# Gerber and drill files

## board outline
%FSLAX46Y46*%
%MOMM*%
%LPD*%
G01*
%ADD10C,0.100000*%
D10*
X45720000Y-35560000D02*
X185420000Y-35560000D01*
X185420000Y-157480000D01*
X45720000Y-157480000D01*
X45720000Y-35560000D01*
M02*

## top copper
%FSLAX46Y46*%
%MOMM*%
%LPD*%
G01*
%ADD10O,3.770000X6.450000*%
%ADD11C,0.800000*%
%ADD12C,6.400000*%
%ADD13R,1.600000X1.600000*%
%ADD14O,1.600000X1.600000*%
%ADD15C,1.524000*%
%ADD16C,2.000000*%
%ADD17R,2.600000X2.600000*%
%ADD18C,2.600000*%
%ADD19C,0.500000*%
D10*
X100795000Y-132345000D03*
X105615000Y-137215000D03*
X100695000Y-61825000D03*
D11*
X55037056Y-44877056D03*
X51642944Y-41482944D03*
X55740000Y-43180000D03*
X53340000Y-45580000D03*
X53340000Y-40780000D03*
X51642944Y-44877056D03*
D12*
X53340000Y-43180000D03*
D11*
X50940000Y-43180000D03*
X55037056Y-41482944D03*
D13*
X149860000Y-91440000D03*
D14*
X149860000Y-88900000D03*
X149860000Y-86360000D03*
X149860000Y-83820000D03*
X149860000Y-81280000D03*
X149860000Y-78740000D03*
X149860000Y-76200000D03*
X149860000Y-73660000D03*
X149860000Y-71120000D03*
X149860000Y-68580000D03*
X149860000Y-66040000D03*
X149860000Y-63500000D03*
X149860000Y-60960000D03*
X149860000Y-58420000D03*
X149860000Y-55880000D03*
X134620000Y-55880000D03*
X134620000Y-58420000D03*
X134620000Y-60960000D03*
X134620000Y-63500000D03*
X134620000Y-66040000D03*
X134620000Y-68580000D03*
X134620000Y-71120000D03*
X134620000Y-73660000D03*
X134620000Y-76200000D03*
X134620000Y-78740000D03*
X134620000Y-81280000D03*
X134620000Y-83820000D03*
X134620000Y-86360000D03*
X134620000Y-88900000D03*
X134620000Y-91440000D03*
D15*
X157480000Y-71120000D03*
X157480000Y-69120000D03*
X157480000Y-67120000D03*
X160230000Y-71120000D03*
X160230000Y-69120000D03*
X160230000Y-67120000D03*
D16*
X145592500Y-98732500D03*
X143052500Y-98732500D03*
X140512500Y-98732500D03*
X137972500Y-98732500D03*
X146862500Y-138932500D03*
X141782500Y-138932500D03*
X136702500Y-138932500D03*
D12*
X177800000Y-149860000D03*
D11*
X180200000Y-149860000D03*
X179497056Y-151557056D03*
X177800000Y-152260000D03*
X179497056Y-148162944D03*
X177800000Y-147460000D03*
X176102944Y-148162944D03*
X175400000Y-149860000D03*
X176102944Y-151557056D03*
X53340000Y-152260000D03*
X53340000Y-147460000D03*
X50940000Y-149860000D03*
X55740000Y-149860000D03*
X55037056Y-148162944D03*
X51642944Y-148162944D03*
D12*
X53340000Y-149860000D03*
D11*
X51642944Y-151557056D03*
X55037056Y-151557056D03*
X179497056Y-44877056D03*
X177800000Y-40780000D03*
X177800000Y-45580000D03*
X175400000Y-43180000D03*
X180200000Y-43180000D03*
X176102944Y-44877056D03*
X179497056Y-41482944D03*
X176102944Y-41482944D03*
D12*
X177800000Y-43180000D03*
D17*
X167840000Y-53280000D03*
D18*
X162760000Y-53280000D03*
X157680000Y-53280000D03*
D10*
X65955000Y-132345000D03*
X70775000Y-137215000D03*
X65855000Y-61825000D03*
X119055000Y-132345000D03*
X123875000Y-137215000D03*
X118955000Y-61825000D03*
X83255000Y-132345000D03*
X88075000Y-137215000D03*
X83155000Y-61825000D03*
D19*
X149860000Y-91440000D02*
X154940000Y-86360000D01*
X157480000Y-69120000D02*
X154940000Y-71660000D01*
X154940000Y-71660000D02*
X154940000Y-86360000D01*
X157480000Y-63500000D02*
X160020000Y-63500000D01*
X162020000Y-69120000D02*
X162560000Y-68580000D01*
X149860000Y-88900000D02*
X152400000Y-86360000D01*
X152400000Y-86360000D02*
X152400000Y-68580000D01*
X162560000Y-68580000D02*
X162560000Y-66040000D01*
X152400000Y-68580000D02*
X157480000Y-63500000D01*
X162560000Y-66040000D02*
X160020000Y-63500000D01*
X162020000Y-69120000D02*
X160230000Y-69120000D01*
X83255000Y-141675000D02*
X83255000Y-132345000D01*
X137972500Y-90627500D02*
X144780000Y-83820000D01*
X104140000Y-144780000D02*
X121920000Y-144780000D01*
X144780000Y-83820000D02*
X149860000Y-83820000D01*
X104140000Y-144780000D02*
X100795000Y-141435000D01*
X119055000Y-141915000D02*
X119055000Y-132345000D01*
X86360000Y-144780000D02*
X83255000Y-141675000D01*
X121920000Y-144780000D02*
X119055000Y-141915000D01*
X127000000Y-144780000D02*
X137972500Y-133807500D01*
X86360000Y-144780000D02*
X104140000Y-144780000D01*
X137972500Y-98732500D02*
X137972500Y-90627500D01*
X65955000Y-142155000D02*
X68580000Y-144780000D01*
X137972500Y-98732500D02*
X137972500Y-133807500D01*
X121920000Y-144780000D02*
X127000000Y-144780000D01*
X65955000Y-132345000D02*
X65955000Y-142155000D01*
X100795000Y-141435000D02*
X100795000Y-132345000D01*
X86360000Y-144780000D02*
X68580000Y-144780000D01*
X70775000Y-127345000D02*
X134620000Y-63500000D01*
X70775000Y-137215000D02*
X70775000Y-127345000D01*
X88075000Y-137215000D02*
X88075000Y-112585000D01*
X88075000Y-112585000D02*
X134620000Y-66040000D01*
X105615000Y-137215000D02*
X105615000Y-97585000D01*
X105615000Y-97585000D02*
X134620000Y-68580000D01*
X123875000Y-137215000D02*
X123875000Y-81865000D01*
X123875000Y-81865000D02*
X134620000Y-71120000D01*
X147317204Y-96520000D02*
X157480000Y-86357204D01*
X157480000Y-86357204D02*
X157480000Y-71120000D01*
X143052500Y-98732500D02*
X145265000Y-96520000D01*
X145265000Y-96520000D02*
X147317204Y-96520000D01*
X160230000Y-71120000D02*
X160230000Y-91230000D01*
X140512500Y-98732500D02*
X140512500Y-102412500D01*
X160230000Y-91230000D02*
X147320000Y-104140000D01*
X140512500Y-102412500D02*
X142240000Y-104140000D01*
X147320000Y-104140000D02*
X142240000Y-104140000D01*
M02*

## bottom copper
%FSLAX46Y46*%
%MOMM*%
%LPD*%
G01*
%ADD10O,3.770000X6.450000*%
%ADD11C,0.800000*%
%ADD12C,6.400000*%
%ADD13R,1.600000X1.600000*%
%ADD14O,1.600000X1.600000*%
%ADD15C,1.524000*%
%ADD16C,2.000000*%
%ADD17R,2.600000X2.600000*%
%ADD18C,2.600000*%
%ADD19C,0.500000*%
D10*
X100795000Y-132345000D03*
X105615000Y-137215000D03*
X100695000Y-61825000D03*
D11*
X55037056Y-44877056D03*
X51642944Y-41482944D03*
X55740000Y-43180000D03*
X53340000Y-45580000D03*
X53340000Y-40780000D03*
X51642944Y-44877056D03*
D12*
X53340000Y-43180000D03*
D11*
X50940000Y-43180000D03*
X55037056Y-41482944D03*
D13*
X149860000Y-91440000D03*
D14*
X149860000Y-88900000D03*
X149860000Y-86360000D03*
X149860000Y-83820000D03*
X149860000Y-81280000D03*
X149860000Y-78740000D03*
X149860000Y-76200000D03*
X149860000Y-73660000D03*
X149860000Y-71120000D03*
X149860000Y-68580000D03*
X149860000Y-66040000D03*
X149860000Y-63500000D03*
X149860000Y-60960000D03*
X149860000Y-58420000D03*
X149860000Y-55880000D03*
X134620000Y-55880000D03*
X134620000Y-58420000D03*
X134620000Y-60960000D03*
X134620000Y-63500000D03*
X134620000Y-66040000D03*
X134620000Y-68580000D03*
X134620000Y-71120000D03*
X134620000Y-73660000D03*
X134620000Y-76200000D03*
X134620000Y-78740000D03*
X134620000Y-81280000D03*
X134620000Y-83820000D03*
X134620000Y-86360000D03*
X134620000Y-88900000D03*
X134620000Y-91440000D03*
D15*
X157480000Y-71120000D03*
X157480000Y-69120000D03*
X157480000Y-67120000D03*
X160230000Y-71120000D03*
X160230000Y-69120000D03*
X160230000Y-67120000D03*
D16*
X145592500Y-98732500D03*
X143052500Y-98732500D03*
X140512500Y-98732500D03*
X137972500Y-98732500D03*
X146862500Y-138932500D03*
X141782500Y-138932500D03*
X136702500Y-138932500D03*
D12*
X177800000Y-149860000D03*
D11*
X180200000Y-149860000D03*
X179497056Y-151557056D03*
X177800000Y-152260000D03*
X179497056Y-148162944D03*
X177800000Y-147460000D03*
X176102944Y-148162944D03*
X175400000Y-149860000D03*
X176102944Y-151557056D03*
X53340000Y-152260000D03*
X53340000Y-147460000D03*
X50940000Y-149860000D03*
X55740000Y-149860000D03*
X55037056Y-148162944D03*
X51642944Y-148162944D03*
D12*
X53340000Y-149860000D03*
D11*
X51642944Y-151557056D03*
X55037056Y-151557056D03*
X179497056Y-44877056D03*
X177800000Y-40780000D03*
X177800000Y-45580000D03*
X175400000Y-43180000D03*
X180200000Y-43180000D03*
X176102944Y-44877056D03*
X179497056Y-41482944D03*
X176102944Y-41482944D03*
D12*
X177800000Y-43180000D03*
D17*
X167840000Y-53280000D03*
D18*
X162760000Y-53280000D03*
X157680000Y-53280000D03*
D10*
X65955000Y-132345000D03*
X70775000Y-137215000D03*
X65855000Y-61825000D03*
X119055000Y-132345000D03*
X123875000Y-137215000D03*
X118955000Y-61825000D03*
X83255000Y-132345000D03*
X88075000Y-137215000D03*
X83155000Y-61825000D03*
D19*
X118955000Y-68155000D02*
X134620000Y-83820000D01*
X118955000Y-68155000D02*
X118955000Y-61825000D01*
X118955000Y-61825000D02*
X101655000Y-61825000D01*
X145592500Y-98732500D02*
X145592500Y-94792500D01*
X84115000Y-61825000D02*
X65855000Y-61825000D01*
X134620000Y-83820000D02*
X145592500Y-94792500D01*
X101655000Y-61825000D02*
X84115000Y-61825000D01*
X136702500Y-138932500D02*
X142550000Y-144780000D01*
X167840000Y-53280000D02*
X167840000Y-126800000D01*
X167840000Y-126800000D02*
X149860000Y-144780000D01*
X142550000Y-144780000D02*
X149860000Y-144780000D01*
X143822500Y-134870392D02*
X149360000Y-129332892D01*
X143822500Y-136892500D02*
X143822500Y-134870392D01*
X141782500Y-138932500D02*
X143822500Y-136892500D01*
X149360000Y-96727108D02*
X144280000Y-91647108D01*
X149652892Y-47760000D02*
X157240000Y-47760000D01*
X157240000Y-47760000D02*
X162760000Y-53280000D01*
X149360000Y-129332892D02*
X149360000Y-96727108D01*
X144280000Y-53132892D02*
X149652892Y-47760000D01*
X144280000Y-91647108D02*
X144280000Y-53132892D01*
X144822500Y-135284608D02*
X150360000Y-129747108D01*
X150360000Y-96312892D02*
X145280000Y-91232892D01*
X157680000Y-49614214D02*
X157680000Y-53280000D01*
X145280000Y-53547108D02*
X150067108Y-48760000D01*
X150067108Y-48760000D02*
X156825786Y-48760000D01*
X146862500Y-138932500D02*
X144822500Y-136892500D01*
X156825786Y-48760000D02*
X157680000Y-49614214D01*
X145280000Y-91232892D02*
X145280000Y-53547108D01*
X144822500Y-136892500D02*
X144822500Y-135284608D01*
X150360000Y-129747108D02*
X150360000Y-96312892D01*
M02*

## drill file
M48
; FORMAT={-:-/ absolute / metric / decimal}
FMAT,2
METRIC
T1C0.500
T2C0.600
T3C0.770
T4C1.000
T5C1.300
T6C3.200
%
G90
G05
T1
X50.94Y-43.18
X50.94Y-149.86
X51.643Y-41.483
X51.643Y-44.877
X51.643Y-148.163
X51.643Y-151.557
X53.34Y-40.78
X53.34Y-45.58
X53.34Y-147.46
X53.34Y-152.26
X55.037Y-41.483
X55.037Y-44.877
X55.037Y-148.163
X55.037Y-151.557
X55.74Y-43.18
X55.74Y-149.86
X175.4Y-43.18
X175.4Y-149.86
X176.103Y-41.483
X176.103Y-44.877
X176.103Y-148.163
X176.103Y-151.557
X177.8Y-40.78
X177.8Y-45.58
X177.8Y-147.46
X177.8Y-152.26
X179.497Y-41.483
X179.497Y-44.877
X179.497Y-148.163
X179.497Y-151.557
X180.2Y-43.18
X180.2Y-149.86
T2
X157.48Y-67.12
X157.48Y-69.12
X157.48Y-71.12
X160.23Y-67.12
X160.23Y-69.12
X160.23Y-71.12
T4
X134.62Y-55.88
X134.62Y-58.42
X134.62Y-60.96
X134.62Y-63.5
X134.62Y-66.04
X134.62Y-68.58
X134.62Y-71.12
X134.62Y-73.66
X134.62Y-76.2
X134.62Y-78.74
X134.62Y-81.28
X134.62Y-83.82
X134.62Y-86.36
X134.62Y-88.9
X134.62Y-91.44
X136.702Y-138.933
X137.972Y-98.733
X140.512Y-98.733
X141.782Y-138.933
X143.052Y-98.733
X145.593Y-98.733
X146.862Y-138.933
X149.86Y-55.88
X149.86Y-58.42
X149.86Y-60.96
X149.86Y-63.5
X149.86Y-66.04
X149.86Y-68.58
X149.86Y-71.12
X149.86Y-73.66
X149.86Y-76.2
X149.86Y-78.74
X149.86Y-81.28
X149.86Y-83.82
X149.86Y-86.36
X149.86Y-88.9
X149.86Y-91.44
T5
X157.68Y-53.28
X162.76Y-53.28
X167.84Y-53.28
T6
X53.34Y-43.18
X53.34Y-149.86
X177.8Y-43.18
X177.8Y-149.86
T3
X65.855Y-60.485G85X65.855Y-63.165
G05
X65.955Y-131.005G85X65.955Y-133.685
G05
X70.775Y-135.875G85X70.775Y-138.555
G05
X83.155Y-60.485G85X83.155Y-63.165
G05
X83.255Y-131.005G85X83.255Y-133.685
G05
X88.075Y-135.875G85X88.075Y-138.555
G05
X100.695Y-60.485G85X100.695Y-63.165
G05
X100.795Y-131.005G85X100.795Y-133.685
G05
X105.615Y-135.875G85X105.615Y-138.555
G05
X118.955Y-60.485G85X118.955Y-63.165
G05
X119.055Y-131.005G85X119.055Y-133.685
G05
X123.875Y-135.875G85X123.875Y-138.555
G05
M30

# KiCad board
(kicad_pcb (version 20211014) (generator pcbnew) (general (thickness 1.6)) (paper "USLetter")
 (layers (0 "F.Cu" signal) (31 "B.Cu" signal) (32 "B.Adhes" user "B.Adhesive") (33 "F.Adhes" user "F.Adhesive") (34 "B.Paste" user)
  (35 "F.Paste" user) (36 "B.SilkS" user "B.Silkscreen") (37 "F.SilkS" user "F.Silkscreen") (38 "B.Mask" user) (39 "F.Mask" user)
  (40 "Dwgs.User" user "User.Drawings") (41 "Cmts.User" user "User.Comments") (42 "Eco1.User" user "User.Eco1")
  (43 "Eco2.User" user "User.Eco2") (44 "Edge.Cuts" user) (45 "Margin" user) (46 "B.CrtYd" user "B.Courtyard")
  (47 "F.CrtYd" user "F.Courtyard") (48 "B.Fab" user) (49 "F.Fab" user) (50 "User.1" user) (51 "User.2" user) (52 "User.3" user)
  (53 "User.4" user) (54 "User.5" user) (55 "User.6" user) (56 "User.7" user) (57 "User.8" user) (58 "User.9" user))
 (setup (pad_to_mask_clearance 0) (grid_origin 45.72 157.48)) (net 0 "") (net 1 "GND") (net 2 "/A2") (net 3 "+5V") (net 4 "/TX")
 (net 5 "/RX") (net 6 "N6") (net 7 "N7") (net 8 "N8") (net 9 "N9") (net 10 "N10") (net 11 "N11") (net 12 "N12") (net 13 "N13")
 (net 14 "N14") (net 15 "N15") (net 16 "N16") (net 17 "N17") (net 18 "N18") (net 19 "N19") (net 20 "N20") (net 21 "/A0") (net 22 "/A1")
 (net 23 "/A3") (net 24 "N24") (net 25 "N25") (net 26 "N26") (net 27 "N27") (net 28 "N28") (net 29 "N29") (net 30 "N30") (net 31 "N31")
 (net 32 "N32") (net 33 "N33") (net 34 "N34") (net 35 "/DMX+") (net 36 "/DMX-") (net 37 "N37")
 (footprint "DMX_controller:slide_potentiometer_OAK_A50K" (layer "F.Cu") (at 96.225 52.345)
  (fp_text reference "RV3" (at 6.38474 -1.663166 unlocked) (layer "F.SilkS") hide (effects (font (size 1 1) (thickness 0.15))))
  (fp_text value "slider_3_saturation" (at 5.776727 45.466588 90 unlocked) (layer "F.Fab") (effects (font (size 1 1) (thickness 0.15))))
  (pad "1" thru_hole oval (at 4.57 80) (size 3.77 6.45) (drill oval 0.77 3.45) (layers *.Cu *.Mask) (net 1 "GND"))
  (pad "2" thru_hole oval (at 9.39 84.87) (size 3.77 6.45) (drill oval 0.77 3.45) (layers *.Cu *.Mask) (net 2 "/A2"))
  (pad "3" thru_hole oval (at 4.47 9.48) (size 3.77 6.45) (drill oval 0.77 3.45) (layers *.Cu *.Mask) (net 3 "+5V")))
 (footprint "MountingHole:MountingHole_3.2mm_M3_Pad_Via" (layer "F.Cu") (at 53.34 43.18)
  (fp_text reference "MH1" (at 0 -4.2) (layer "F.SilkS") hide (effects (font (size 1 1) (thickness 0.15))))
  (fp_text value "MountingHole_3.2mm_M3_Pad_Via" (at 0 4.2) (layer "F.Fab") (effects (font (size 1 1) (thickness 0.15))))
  (pad "1" thru_hole circle (at 1.697056 1.697056) (size 0.8 0.8) (drill 0.5) (layers *.Cu *.Mask))
  (pad "1" thru_hole circle (at -1.697056 -1.697056) (size 0.8 0.8) (drill 0.5) (layers *.Cu *.Mask))
  (pad "1" thru_hole circle (at 2.4 0) (size 0.8 0.8) (drill 0.5) (layers *.Cu *.Mask))
  (pad "1" thru_hole circle (at 0 2.4) (size 0.8 0.8) (drill 0.5) (layers *.Cu *.Mask))
  (pad "1" thru_hole circle (at 0 -2.4) (size 0.8 0.8) (drill 0.5) (layers *.Cu *.Mask))
  (pad "1" thru_hole circle (at -1.697056 1.697056) (size 0.8 0.8) (drill 0.5) (layers *.Cu *.Mask))
  (pad "1" thru_hole circle (at 0 0) (size 6.4 6.4) (drill 3.2) (layers *.Cu *.Mask))
  (pad "1" thru_hole circle (at -2.4 0) (size 0.8 0.8) (drill 0.5) (layers *.Cu *.Mask))
  (pad "1" thru_hole circle (at 1.697056 -1.697056) (size 0.8 0.8) (drill 0.5) (layers *.Cu *.Mask)))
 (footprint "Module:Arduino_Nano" (layer "F.Cu") (at 149.86 91.44 180)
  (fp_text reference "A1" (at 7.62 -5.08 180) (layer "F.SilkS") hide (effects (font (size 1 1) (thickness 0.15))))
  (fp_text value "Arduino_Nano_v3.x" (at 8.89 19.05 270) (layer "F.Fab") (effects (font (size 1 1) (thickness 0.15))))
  (pad "1" thru_hole rect (at 0 0 180) (size 1.6 1.6) (drill 1) (layers *.Cu *.Mask) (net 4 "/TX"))
  (pad "2" thru_hole oval (at 0 2.54 180) (size 1.6 1.6) (drill 1) (layers *.Cu *.Mask) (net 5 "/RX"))
  (pad "3" thru_hole oval (at 0 5.08 180) (size 1.6 1.6) (drill 1) (layers *.Cu *.Mask) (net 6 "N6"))
  (pad "4" thru_hole oval (at 0 7.62 180) (size 1.6 1.6) (drill 1) (layers *.Cu *.Mask) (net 1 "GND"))
  (pad "5" thru_hole oval (at 0 10.16 180) (size 1.6 1.6) (drill 1) (layers *.Cu *.Mask) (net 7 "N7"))
  (pad "6" thru_hole oval (at 0 12.7 180) (size 1.6 1.6) (drill 1) (layers *.Cu *.Mask) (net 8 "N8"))
  (pad "7" thru_hole oval (at 0 15.24 180) (size 1.6 1.6) (drill 1) (layers *.Cu *.Mask) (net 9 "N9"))
  (pad "8" thru_hole oval (at 0 17.78 180) (size 1.6 1.6) (drill 1) (layers *.Cu *.Mask) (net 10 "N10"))
  (pad "9" thru_hole oval (at 0 20.32 180) (size 1.6 1.6) (drill 1) (layers *.Cu *.Mask) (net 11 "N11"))
  (pad "10" thru_hole oval (at 0 22.86 180) (size 1.6 1.6) (drill 1) (layers *.Cu *.Mask) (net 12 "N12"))
  (pad "11" thru_hole oval (at 0 25.4 180) (size 1.6 1.6) (drill 1) (layers *.Cu *.Mask) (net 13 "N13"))
  (pad "12" thru_hole oval (at 0 27.94 180) (size 1.6 1.6) (drill 1) (layers *.Cu *.Mask) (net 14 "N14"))
  (pad "13" thru_hole oval (at 0 30.48 180) (size 1.6 1.6) (drill 1) (layers *.Cu *.Mask) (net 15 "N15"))
  (pad "14" thru_hole oval (at 0 33.02 180) (size 1.6 1.6) (drill 1) (layers *.Cu *.Mask) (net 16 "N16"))
  (pad "15" thru_hole oval (at 0 35.56 180) (size 1.6 1.6) (drill 1) (layers *.Cu *.Mask) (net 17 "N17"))
  (pad "16" thru_hole oval (at 15.24 35.56 180) (size 1.6 1.6) (drill 1) (layers *.Cu *.Mask) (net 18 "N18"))
  (pad "17" thru_hole oval (at 15.24 33.02 180) (size 1.6 1.6) (drill 1) (layers *.Cu *.Mask) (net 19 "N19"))
  (pad "18" thru_hole oval (at 15.24 30.48 180) (size 1.6 1.6) (drill 1) (layers *.Cu *.Mask) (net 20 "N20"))
  (pad "19" thru_hole oval (at 15.24 27.94 180) (size 1.6 1.6) (drill 1) (layers *.Cu *.Mask) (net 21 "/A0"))
  (pad "20" thru_hole oval (at 15.24 25.4 180) (size 1.6 1.6) (drill 1) (layers *.Cu *.Mask) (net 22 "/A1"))
  (pad "21" thru_hole oval (at 15.24 22.86 180) (size 1.6 1.6) (drill 1) (layers *.Cu *.Mask) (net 2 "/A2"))
  (pad "22" thru_hole oval (at 15.24 20.32 180) (size 1.6 1.6) (drill 1) (layers *.Cu *.Mask) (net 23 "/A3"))
  (pad "23" thru_hole oval (at 15.24 17.78 180) (size 1.6 1.6) (drill 1) (layers *.Cu *.Mask) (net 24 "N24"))
  (pad "24" thru_hole oval (at 15.24 15.24 180) (size 1.6 1.6) (drill 1) (layers *.Cu *.Mask) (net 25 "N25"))
  (pad "25" thru_hole oval (at 15.24 12.7 180) (size 1.6 1.6) (drill 1) (layers *.Cu *.Mask) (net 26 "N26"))
  (pad "26" thru_hole oval (at 15.24 10.16 180) (size 1.6 1.6) (drill 1) (layers *.Cu *.Mask) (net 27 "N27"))
  (pad "27" thru_hole oval (at 15.24 7.62 180) (size 1.6 1.6) (drill 1) (layers *.Cu *.Mask) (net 3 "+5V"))
  (pad "28" thru_hole oval (at 15.24 5.08 180) (size 1.6 1.6) (drill 1) (layers *.Cu *.Mask) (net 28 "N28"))
  (pad "29" thru_hole oval (at 15.24 2.54 180) (size 1.6 1.6) (drill 1) (layers *.Cu *.Mask) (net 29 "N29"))
  (pad "30" thru_hole oval (at 15.24 0 180) (size 1.6 1.6) (drill 1) (layers *.Cu *.Mask) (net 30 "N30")))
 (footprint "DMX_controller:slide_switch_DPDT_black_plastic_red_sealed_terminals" (layer "F.Cu") (at 157.48 71.12 90)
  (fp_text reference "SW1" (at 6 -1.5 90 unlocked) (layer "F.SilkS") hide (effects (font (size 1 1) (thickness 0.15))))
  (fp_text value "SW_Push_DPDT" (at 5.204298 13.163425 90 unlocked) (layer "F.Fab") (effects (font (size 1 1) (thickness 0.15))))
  (pad "1" thru_hole circle (at 0 0 90) (size 1.524 1.524) (drill 0.6) (layers *.Cu *.Mask) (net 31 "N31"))
  (pad "2" thru_hole circle (at 2 0 90) (size 1.524 1.524) (drill 0.6) (layers *.Cu *.Mask) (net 4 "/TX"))
  (pad "3" thru_hole circle (at 4 0 90) (size 1.524 1.524) (drill 0.6) (layers *.Cu *.Mask) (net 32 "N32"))
  (pad "4" thru_hole circle (at 0 2.75 90) (size 1.524 1.524) (drill 0.6) (layers *.Cu *.Mask) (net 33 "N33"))
  (pad "5" thru_hole circle (at 2 2.75 90) (size 1.524 1.524) (drill 0.6) (layers *.Cu *.Mask) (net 5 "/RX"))
  (pad "6" thru_hole circle (at 4 2.75 90) (size 1.524 1.524) (drill 0.6) (layers *.Cu *.Mask) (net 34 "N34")))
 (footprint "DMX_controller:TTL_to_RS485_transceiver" (layer "F.Cu") (at 145.5925 98.7325 -90)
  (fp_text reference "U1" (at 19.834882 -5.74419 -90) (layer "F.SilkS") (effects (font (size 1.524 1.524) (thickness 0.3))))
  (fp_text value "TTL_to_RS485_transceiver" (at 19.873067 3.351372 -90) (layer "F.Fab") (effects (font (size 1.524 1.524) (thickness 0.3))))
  (pad "1" thru_hole circle (at 0 0 180) (size 2 2) (drill 1) (layers *.Cu *.Mask) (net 3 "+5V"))
  (pad "2" thru_hole circle (at 0 2.54 180) (size 2 2) (drill 1) (layers *.Cu *.Mask) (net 31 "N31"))
  (pad "3" thru_hole circle (at 0 5.08 180) (size 2 2) (drill 1) (layers *.Cu *.Mask) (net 33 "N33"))
  (pad "4" thru_hole circle (at 0 7.62 180) (size 2 2) (drill 1) (layers *.Cu *.Mask) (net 1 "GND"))
  (pad "5" thru_hole circle (at 40.2 -1.27 180) (size 2 2) (drill 1) (layers *.Cu *.Mask) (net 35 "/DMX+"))
  (pad "6" thru_hole circle (at 40.2 3.81 180) (size 2 2) (drill 1) (layers *.Cu *.Mask) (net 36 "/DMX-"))
  (pad "7" thru_hole circle (at 40.2 8.89 180) (size 2 2) (drill 1) (layers *.Cu *.Mask) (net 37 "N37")))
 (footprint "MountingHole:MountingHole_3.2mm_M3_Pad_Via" (layer "F.Cu") (at 177.8 149.86)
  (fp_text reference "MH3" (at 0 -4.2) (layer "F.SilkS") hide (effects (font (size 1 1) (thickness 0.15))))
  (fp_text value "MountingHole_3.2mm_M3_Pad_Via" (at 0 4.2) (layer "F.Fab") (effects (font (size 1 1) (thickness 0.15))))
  (pad "1" thru_hole circle (at 0 0) (size 6.4 6.4) (drill 3.2) (layers *.Cu *.Mask))
  (pad "1" thru_hole circle (at 2.4 0) (size 0.8 0.8) (drill 0.5) (layers *.Cu *.Mask))
  (pad "1" thru_hole circle (at 1.697056 1.697056) (size 0.8 0.8) (drill 0.5) (layers *.Cu *.Mask))
  (pad "1" thru_hole circle (at 0 2.4) (size 0.8 0.8) (drill 0.5) (layers *.Cu *.Mask))
  (pad "1" thru_hole circle (at 1.697056 -1.697056) (size 0.8 0.8) (drill 0.5) (layers *.Cu *.Mask))
  (pad "1" thru_hole circle (at 0 -2.4) (size 0.8 0.8) (drill 0.5) (layers *.Cu *.Mask))
  (pad "1" thru_hole circle (at -1.697056 -1.697056) (size 0.8 0.8) (drill 0.5) (layers *.Cu *.Mask))
  (pad "1" thru_hole circle (at -2.4 0) (size 0.8 0.8) (drill 0.5) (layers *.Cu *.Mask))
  (pad "1" thru_hole circle (at -1.697056 1.697056) (size 0.8 0.8) (drill 0.5) (layers *.Cu *.Mask)))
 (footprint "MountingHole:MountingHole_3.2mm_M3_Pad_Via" (layer "F.Cu") (at 53.34 149.86)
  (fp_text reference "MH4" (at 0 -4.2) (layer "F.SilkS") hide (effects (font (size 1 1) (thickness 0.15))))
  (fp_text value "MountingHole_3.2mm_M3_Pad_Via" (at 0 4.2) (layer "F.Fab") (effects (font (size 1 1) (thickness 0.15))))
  (pad "1" thru_hole circle (at 0 2.4) (size 0.8 0.8) (drill 0.5) (layers *.Cu *.Mask))
  (pad "1" thru_hole circle (at 0 -2.4) (size 0.8 0.8) (drill 0.5) (layers *.Cu *.Mask))
  (pad "1" thru_hole circle (at -2.4 0) (size 0.8 0.8) (drill 0.5) (layers *.Cu *.Mask))
  (pad "1" thru_hole circle (at 2.4 0) (size 0.8 0.8) (drill 0.5) (layers *.Cu *.Mask))
  (pad "1" thru_hole circle (at 1.697056 -1.697056) (size 0.8 0.8) (drill 0.5) (layers *.Cu *.Mask))
  (pad "1" thru_hole circle (at -1.697056 -1.697056) (size 0.8 0.8) (drill 0.5) (layers *.Cu *.Mask))
  (pad "1" thru_hole circle (at 0 0) (size 6.4 6.4) (drill 3.2) (layers *.Cu *.Mask))
  (pad "1" thru_hole circle (at -1.697056 1.697056) (size 0.8 0.8) (drill 0.5) (layers *.Cu *.Mask))
  (pad "1" thru_hole circle (at 1.697056 1.697056) (size 0.8 0.8) (drill 0.5) (layers *.Cu *.Mask)))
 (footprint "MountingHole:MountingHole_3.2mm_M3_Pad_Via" (layer "F.Cu") (at 177.8 43.18)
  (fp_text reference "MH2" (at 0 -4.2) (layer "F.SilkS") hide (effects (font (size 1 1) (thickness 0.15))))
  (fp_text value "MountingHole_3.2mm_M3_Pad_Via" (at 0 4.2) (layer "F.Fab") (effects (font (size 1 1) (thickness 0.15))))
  (pad "1" thru_hole circle (at 1.697056 1.697056) (size 0.8 0.8) (drill 0.5) (layers *.Cu *.Mask))
  (pad "1" thru_hole circle (at 0 -2.4) (size 0.8 0.8) (drill 0.5) (layers *.Cu *.Mask))
  (pad "1" thru_hole circle (at 0 2.4) (size 0.8 0.8) (drill 0.5) (layers *.Cu *.Mask))
  (pad "1" thru_hole circle (at -2.4 0) (size 0.8 0.8) (drill 0.5) (layers *.Cu *.Mask))
  (pad "1" thru_hole circle (at 2.4 0) (size 0.8 0.8) (drill 0.5) (layers *.Cu *.Mask))
  (pad "1" thru_hole circle (at -1.697056 1.697056) (size 0.8 0.8) (drill 0.5) (layers *.Cu *.Mask))
  (pad "1" thru_hole circle (at 1.697056 -1.697056) (size 0.8 0.8) (drill 0.5) (layers *.Cu *.Mask))
  (pad "1" thru_hole circle (at -1.697056 -1.697056) (size 0.8 0.8) (drill 0.5) (layers *.Cu *.Mask))
  (pad "1" thru_hole circle (at 0 0) (size 6.4 6.4) (drill 3.2) (layers *.Cu *.Mask)))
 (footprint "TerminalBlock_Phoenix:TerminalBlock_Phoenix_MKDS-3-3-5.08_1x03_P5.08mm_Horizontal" (layer "F.Cu") (at 167.84 53.28 180)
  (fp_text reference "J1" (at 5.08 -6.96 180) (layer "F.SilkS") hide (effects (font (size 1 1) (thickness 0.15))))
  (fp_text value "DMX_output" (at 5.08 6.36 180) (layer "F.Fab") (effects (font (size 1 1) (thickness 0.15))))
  (pad "1" thru_hole rect (at 0 0 180) (size 2.6 2.6) (drill 1.3) (layers *.Cu *.Mask) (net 37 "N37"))
  (pad "2" thru_hole circle (at 5.08 0 180) (size 2.6 2.6) (drill 1.3) (layers *.Cu *.Mask) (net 36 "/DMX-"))
  (pad "3" thru_hole circle (at 10.16 0 180) (size 2.6 2.6) (drill 1.3) (layers *.Cu *.Mask) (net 35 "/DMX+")))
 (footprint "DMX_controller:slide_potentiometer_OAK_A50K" (layer "F.Cu") (at 61.385 52.345)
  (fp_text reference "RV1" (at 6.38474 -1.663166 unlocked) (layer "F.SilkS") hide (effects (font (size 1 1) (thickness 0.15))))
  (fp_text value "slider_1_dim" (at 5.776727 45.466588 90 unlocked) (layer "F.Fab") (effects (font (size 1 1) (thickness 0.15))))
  (pad "1" thru_hole oval (at 4.57 80) (size 3.77 6.45) (drill oval 0.77 3.45) (layers *.Cu *.Mask) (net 1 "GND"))
  (pad "2" thru_hole oval (at 9.39 84.87) (size 3.77 6.45) (drill oval 0.77 3.45) (layers *.Cu *.Mask) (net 21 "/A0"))
  (pad "3" thru_hole oval (at 4.47 9.48) (size 3.77 6.45) (drill oval 0.77 3.45) (layers *.Cu *.Mask) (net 3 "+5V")))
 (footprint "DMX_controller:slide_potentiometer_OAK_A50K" (layer "F.Cu") (at 114.485 52.345)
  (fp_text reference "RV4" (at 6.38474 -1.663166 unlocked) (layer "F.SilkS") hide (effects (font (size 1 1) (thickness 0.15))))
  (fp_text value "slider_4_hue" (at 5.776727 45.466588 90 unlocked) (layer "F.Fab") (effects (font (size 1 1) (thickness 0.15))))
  (pad "1" thru_hole oval (at 4.57 80) (size 3.77 6.45) (drill oval 0.77 3.45) (layers *.Cu *.Mask) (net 1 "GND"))
  (pad "2" thru_hole oval (at 9.39 84.87) (size 3.77 6.45) (drill oval 0.77 3.45) (layers *.Cu *.Mask) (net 23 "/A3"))
  (pad "3" thru_hole oval (at 4.47 9.48) (size 3.77 6.45) (drill oval 0.77 3.45) (layers *.Cu *.Mask) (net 3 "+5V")))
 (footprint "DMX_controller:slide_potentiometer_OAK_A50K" (layer "F.Cu") (at 78.685 52.345)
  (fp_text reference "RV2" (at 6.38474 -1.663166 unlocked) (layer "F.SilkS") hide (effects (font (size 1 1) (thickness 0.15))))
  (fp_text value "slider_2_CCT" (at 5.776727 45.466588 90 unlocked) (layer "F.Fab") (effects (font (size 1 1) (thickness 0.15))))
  (pad "1" thru_hole oval (at 4.57 80) (size 3.77 6.45) (drill oval 0.77 3.45) (layers *.Cu *.Mask) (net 1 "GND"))
  (pad "2" thru_hole oval (at 9.39 84.87) (size 3.77 6.45) (drill oval 0.77 3.45) (layers *.Cu *.Mask) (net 22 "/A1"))
  (pad "3" thru_hole oval (at 4.47 9.48) (size 3.77 6.45) (drill oval 0.77 3.45) (layers *.Cu *.Mask) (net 3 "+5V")))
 (gr_rect (start 45.72 35.56) (end 185.42 157.48) (layer "Edge.Cuts") (width 0.1) (fill none))
 (segment (start 149.86 91.44) (end 154.94 86.36) (width 0.5) (layer "F.Cu") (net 4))
 (segment (start 157.48 69.12) (end 154.94 71.66) (width 0.5) (layer "F.Cu") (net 4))
 (segment (start 154.94 71.66) (end 154.94 86.36) (width 0.5) (layer "F.Cu") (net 4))
 (segment (start 157.48 63.5) (end 160.02 63.5) (width 0.5) (layer "F.Cu") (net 5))
 (segment (start 162.02 69.12) (end 162.56 68.58) (width 0.5) (layer "F.Cu") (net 5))
 (segment (start 149.86 88.9) (end 152.4 86.36) (width 0.5) (layer "F.Cu") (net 5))
 (segment (start 152.4 86.36) (end 152.4 68.58) (width 0.5) (layer "F.Cu") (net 5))
 (segment (start 162.56 68.58) (end 162.56 66.04) (width 0.5) (layer "F.Cu") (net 5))
 (segment (start 152.4 68.58) (end 157.48 63.5) (width 0.5) (layer "F.Cu") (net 5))
 (segment (start 162.56 66.04) (end 160.02 63.5) (width 0.5) (layer "F.Cu") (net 5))
 (segment (start 162.02 69.12) (end 160.23 69.12) (width 0.5) (layer "F.Cu") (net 5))
 (segment (start 83.255 141.675) (end 83.255 132.345) (width 0.5) (layer "F.Cu") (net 1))
 (segment (start 137.9725 90.6275) (end 144.78 83.82) (width 0.5) (layer "F.Cu") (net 1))
 (segment (start 104.14 144.78) (end 121.92 144.78) (width 0.5) (layer "F.Cu") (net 1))
 (segment (start 144.78 83.82) (end 149.86 83.82) (width 0.5) (layer "F.Cu") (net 1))
 (segment (start 104.14 144.78) (end 100.795 141.435) (width 0.5) (layer "F.Cu") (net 1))
 (segment (start 119.055 141.915) (end 119.055 132.345) (width 0.5) (layer "F.Cu") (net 1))
 (segment (start 86.36 144.78) (end 83.255 141.675) (width 0.5) (layer "F.Cu") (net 1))
 (segment (start 121.92 144.78) (end 119.055 141.915) (width 0.5) (layer "F.Cu") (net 1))
 (segment (start 127 144.78) (end 137.9725 133.8075) (width 0.5) (layer "F.Cu") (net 1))
 (segment (start 86.36 144.78) (end 104.14 144.78) (width 0.5) (layer "F.Cu") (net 1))
 (segment (start 137.9725 98.7325) (end 137.9725 90.6275) (width 0.5) (layer "F.Cu") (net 1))
 (segment (start 65.955 142.155) (end 68.58 144.78) (width 0.5) (layer "F.Cu") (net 1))
 (segment (start 137.9725 98.7325) (end 137.9725 133.8075) (width 0.5) (layer "F.Cu") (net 1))
 (segment (start 121.92 144.78) (end 127 144.78) (width 0.5) (layer "F.Cu") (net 1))
 (segment (start 65.955 132.345) (end 65.955 142.155) (width 0.5) (layer "F.Cu") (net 1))
 (segment (start 100.795 141.435) (end 100.795 132.345) (width 0.5) (layer "F.Cu") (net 1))
 (segment (start 86.36 144.78) (end 68.58 144.78) (width 0.5) (layer "F.Cu") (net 1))
 (segment (start 70.775 127.345) (end 134.62 63.5) (width 0.5) (layer "F.Cu") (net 21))
 (segment (start 70.775 137.215) (end 70.775 127.345) (width 0.5) (layer "F.Cu") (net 21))
 (segment (start 88.075 137.215) (end 88.075 112.585) (width 0.5) (layer "F.Cu") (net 22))
 (segment (start 88.075 112.585) (end 134.62 66.04) (width 0.5) (layer "F.Cu") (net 22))
 (segment (start 105.615 137.215) (end 105.615 97.585) (width 0.5) (layer "F.Cu") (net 2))
 (segment (start 105.615 97.585) (end 134.62 68.58) (width 0.5) (layer "F.Cu") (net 2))
 (segment (start 123.875 137.215) (end 123.875 81.865) (width 0.5) (layer "F.Cu") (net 23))
 (segment (start 123.875 81.865) (end 134.62 71.12) (width 0.5) (layer "F.Cu") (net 23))
 (segment (start 118.955 68.155) (end 134.62 83.82) (width 0.5) (layer "B.Cu") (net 3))
 (segment (start 118.955 68.155) (end 118.955 61.825) (width 0.5) (layer "B.Cu") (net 3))
 (segment (start 118.955 61.825) (end 101.655 61.825) (width 0.5) (layer "B.Cu") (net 3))
 (segment (start 145.5925 98.7325) (end 145.5925 94.7925) (width 0.5) (layer "B.Cu") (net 3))
 (segment (start 84.115 61.825) (end 65.855 61.825) (width 0.5) (layer "B.Cu") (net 3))
 (segment (start 134.62 83.82) (end 145.5925 94.7925) (width 0.5) (layer "B.Cu") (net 3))
 (segment (start 101.655 61.825) (end 84.115 61.825) (width 0.5) (layer "B.Cu") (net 3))
 (segment (start 136.7025 138.9325) (end 142.55 144.78) (width 0.5) (layer "B.Cu") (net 37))
 (segment (start 167.84 53.28) (end 167.84 126.8) (width 0.5) (layer "B.Cu") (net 37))
 (segment (start 167.84 126.8) (end 149.86 144.78) (width 0.5) (layer "B.Cu") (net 37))
 (segment (start 142.55 144.78) (end 149.86 144.78) (width 0.5) (layer "B.Cu") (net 37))
 (segment (start 143.8225 134.870392) (end 149.36 129.332892) (width 0.5) (layer "B.Cu") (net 36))
 (segment (start 143.8225 136.8925) (end 143.8225 134.870392) (width 0.5) (layer "B.Cu") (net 36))
 (segment (start 141.7825 138.9325) (end 143.8225 136.8925) (width 0.5) (layer "B.Cu") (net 36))
 (segment (start 149.36 96.727108) (end 144.28 91.647108) (width 0.5) (layer "B.Cu") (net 36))
 (segment (start 149.652892 47.76) (end 157.24 47.76) (width 0.5) (layer "B.Cu") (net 36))
 (segment (start 157.24 47.76) (end 162.76 53.28) (width 0.5) (layer "B.Cu") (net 36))
 (segment (start 149.36 129.332892) (end 149.36 96.727108) (width 0.5) (layer "B.Cu") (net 36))
 (segment (start 144.28 53.132892) (end 149.652892 47.76) (width 0.5) (layer "B.Cu") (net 36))
 (segment (start 144.28 91.647108) (end 144.28 53.132892) (width 0.5) (layer "B.Cu") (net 36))
 (segment (start 144.8225 135.284608) (end 150.36 129.747108) (width 0.5) (layer "B.Cu") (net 35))
 (segment (start 150.36 96.312892) (end 145.28 91.232892) (width 0.5) (layer "B.Cu") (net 35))
 (segment (start 157.68 49.614214) (end 157.68 53.28) (width 0.5) (layer "B.Cu") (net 35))
 (segment (start 145.28 53.547108) (end 150.067108 48.76) (width 0.5) (layer "B.Cu") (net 35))
 (segment (start 150.067108 48.76) (end 156.825786 48.76) (width 0.5) (layer "B.Cu") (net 35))
 (segment (start 146.8625 138.9325) (end 144.8225 136.8925) (width 0.5) (layer "B.Cu") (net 35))
 (segment (start 156.825786 48.76) (end 157.68 49.614214) (width 0.5) (layer "B.Cu") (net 35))
 (segment (start 145.28 91.232892) (end 145.28 53.547108) (width 0.5) (layer "B.Cu") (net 35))
 (segment (start 144.8225 136.8925) (end 144.8225 135.284608) (width 0.5) (layer "B.Cu") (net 35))
 (segment (start 150.36 129.747108) (end 150.36 96.312892) (width 0.5) (layer "B.Cu") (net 35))
 (segment (start 147.317204 96.52) (end 157.48 86.357204) (width 0.5) (layer "F.Cu") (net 31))
 (segment (start 157.48 86.357204) (end 157.48 71.12) (width 0.5) (layer "F.Cu") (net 31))
 (segment (start 143.0525 98.7325) (end 145.265 96.52) (width 0.5) (layer "F.Cu") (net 31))
 (segment (start 145.265 96.52) (end 147.317204 96.52) (width 0.5) (layer "F.Cu") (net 31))
 (segment (start 160.23 71.12) (end 160.23 91.23) (width 0.5) (layer "F.Cu") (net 33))
 (segment (start 140.5125 98.7325) (end 140.5125 102.4125) (width 0.5) (layer "F.Cu") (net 33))
 (segment (start 160.23 91.23) (end 147.32 104.14) (width 0.5) (layer "F.Cu") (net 33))
 (segment (start 140.5125 102.4125) (end 142.24 104.14) (width 0.5) (layer "F.Cu") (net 33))
 (segment (start 147.32 104.14) (end 142.24 104.14) (width 0.5) (layer "F.Cu") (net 33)))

